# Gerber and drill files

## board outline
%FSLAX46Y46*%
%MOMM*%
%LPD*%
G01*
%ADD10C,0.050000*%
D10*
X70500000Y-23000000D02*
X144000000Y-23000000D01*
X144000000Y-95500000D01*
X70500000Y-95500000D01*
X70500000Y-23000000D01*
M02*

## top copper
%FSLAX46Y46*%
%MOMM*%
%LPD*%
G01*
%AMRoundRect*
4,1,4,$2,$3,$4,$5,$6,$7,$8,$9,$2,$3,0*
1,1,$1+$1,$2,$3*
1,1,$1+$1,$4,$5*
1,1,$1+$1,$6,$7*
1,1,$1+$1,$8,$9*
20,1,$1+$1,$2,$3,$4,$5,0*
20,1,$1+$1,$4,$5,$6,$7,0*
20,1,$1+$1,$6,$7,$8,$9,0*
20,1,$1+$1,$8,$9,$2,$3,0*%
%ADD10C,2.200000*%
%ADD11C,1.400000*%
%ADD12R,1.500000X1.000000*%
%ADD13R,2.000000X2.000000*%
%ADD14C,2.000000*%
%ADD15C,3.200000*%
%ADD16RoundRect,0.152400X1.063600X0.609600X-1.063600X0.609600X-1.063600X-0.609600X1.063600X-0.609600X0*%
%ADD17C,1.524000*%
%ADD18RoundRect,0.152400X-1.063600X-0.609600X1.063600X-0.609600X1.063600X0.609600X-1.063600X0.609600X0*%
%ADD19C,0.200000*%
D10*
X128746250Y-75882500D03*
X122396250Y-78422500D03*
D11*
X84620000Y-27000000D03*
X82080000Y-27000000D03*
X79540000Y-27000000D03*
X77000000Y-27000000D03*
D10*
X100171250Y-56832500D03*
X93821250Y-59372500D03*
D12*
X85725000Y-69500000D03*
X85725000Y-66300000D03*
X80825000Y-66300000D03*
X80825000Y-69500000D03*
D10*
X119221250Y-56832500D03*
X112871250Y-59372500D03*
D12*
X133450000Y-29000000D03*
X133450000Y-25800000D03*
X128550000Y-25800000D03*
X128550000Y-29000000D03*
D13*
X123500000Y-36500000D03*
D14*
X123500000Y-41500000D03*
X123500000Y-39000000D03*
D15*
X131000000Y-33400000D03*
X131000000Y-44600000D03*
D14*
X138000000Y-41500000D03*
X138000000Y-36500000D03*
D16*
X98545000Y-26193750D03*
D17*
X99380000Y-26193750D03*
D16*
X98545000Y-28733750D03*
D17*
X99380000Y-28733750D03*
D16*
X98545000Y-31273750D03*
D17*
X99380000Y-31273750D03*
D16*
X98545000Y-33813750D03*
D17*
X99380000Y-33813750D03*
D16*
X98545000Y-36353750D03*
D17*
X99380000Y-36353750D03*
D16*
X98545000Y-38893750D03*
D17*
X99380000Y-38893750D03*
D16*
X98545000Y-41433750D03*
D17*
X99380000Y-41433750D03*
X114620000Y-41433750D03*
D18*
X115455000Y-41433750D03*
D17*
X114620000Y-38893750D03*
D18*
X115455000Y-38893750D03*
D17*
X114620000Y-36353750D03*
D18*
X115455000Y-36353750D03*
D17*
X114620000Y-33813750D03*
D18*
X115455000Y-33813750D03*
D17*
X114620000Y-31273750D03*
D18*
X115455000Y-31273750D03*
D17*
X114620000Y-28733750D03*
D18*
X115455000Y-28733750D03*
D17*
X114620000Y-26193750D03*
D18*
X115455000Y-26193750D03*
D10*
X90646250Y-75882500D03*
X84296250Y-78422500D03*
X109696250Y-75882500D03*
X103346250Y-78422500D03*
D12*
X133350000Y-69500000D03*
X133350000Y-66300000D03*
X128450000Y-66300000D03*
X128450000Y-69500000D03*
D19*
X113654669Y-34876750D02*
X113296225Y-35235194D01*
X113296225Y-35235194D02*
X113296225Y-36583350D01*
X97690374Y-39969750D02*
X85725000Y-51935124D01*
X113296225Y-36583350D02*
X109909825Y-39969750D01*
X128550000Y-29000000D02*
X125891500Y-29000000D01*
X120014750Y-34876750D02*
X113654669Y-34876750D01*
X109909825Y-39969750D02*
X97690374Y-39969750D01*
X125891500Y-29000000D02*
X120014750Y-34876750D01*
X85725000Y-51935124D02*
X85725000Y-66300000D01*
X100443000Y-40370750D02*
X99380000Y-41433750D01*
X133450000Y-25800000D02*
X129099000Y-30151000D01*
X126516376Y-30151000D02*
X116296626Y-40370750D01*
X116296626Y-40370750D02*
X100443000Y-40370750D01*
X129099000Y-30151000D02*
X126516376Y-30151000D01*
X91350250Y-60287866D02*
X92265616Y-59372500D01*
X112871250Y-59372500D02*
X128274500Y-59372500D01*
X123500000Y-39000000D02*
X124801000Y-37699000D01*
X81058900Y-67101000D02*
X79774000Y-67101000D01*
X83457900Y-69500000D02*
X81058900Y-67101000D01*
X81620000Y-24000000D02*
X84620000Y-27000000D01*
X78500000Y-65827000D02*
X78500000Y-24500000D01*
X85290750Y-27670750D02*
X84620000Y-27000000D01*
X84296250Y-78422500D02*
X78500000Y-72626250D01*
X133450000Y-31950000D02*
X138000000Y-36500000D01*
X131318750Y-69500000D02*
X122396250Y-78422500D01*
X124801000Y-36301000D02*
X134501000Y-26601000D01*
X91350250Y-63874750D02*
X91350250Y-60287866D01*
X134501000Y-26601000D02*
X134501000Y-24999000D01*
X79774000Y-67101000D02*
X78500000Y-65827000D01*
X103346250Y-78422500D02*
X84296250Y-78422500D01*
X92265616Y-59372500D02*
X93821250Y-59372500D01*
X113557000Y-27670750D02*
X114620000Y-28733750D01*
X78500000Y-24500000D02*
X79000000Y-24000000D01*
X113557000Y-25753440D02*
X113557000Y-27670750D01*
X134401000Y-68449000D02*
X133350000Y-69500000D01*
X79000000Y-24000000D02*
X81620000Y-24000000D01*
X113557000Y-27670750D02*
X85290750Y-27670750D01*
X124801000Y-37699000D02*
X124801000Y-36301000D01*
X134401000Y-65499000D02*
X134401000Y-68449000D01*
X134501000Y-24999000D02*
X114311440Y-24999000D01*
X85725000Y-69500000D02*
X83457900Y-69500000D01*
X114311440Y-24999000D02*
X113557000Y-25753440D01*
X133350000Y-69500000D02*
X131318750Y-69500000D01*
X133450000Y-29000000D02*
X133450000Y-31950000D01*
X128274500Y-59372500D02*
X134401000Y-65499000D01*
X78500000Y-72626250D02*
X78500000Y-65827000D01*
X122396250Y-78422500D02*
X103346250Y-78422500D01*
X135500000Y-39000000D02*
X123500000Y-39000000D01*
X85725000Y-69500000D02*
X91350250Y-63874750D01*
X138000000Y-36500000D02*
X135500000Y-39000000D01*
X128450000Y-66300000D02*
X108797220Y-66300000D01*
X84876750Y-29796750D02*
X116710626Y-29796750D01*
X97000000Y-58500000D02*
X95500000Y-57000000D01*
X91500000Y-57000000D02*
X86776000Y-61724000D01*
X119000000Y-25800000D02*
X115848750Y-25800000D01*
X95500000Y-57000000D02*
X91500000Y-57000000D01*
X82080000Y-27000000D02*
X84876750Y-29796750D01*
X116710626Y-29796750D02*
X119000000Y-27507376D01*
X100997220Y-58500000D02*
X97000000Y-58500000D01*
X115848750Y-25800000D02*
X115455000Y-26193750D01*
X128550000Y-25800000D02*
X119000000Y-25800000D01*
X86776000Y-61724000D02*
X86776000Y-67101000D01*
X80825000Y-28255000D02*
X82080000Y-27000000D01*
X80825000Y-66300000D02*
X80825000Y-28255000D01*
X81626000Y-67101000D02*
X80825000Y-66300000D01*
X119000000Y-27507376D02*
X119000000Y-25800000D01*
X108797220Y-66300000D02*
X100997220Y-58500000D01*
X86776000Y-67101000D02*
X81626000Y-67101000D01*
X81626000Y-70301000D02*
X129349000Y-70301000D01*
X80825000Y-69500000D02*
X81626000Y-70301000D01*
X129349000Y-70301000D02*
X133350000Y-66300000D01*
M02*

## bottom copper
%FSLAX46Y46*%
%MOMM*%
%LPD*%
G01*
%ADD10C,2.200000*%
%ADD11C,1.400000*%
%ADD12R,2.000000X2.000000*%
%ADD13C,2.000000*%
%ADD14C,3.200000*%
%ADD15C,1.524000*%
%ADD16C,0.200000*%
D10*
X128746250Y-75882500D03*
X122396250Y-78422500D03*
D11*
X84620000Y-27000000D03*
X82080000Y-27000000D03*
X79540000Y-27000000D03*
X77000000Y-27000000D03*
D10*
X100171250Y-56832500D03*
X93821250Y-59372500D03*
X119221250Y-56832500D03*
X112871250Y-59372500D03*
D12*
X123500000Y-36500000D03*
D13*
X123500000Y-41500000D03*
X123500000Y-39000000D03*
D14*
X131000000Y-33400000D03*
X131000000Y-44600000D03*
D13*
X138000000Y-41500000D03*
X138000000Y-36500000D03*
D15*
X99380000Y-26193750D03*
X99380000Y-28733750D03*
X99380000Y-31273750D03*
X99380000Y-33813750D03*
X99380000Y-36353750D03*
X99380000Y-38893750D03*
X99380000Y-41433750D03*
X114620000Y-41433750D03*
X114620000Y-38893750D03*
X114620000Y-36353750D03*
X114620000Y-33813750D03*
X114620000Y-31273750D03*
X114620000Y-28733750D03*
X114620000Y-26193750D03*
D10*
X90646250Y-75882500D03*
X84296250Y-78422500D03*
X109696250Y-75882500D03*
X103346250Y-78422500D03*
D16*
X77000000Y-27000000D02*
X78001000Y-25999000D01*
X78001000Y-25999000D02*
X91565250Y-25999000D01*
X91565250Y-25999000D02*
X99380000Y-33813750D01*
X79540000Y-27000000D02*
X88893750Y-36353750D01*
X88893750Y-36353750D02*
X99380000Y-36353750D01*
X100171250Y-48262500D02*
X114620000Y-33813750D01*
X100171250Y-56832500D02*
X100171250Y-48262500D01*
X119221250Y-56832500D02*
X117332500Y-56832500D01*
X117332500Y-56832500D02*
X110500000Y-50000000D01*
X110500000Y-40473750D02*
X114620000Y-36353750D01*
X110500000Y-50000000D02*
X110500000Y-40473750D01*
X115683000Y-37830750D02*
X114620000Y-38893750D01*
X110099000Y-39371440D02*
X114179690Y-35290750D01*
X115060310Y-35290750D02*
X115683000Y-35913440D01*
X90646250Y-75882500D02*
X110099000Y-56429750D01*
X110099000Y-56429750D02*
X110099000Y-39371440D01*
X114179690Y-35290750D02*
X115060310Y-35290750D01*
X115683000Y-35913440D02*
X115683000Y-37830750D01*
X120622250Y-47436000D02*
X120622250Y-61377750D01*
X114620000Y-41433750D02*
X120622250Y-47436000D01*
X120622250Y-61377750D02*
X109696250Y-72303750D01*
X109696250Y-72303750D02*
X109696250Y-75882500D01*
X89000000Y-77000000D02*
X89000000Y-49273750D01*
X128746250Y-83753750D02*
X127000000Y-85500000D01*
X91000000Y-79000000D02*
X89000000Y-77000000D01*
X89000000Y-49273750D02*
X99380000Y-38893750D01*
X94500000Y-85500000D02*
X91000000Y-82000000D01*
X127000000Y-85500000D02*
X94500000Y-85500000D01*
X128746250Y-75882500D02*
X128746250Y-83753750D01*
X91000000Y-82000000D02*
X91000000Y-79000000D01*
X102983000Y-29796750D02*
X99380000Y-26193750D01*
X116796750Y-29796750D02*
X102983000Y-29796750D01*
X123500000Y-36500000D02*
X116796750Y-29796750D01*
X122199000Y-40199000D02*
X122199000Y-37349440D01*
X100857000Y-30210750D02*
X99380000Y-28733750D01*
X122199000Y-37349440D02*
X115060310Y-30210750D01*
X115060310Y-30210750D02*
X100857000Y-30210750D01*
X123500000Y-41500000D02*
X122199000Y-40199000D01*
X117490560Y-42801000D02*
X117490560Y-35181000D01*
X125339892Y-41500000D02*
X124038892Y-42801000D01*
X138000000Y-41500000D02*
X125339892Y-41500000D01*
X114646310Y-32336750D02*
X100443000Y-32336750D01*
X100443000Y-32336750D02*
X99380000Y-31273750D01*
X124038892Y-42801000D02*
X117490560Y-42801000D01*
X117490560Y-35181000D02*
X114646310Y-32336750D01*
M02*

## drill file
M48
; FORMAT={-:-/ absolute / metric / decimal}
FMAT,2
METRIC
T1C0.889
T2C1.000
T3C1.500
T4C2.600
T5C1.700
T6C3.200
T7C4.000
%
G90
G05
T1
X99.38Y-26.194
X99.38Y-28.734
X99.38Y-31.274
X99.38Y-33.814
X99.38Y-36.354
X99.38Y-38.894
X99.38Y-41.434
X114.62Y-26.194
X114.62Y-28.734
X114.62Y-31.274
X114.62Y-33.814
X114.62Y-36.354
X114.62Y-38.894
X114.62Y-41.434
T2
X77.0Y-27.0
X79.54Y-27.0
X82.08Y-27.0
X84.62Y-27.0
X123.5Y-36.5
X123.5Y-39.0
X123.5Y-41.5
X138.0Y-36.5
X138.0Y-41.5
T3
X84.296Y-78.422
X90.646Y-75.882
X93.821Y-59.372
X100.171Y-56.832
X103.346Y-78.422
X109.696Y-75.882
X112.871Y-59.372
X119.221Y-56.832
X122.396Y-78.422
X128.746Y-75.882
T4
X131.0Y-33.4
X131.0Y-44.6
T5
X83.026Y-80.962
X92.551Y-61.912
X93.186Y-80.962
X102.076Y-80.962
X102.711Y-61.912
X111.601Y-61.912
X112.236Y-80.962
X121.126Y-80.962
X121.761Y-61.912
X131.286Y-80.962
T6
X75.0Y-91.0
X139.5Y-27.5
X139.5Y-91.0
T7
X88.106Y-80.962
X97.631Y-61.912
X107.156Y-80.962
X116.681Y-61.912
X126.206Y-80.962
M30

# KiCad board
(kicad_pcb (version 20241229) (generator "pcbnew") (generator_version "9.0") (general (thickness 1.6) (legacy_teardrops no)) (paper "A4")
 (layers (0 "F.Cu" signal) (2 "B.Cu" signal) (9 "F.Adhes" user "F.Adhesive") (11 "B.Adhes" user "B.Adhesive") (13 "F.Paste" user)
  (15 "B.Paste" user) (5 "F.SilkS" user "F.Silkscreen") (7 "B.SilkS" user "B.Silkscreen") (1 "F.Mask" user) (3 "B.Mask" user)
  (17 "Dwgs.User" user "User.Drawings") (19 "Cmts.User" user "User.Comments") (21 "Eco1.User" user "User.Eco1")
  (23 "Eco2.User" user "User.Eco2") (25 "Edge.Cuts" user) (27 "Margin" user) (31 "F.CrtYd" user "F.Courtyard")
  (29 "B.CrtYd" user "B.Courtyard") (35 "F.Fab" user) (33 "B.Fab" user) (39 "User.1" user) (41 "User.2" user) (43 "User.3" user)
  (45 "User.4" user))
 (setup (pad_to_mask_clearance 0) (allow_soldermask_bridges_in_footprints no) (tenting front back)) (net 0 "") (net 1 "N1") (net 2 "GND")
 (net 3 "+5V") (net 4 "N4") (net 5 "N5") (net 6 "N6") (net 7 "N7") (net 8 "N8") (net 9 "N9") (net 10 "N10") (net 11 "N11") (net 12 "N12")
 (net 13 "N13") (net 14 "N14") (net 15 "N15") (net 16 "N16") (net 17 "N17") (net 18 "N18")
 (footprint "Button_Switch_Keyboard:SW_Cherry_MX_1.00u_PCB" (layer "F.Cu") (at 128.74625 75.8825)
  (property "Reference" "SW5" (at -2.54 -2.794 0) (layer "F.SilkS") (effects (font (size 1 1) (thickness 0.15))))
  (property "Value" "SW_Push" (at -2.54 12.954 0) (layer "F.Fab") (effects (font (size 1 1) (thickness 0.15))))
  (pad "" np_thru_hole circle (at -7.62 5.08) (size 1.7 1.7) (drill 1.7) (layers "*.Cu" "*.Mask"))
  (pad "" np_thru_hole circle (at -2.54 5.08) (size 4 4) (drill 4) (layers "*.Cu" "*.Mask"))
  (pad "" np_thru_hole circle (at 2.54 5.08) (size 1.7 1.7) (drill 1.7) (layers "*.Cu" "*.Mask"))
  (pad "1" thru_hole circle (at 0 0) (size 2.2 2.2) (drill 1.5) (layers "*.Cu" "*.Mask") (remove_unused_layers no) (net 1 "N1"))
  (pad "2" thru_hole circle (at -6.35 2.54) (size 2.2 2.2) (drill 1.5) (layers "*.Cu" "*.Mask") (remove_unused_layers no) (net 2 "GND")))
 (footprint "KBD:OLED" (layer "F.Cu") (at 80.81 27 180)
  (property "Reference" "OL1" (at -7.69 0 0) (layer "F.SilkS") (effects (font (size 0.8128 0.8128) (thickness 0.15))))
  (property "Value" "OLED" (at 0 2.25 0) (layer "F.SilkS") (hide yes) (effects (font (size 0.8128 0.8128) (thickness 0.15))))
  (pad "1" thru_hole circle (at -3.81 0 180) (size 1.4 1.4) (drill 1) (layers "*.Cu" "*.Mask") (remove_unused_layers no) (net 2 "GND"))
  (pad "2" thru_hole circle (at -1.27 0 180) (size 1.4 1.4) (drill 1) (layers "*.Cu" "*.Mask") (remove_unused_layers no) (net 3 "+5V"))
  (pad "3" thru_hole circle (at 1.27 0 180) (size 1.4 1.4) (drill 1) (layers "*.Cu" "*.Mask") (remove_unused_layers no) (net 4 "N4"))
  (pad "4" thru_hole circle (at 3.81 0 180) (size 1.4 1.4) (drill 1) (layers "*.Cu" "*.Mask") (remove_unused_layers no) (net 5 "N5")))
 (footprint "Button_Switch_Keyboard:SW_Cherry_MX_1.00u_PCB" (layer "F.Cu") (at 100.17125 56.8325)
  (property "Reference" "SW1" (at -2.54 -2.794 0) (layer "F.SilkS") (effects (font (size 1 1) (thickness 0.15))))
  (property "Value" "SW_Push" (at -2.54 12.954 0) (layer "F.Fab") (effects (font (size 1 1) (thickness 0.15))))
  (pad "" np_thru_hole circle (at -7.62 5.08) (size 1.7 1.7) (drill 1.7) (layers "*.Cu" "*.Mask"))
  (pad "" np_thru_hole circle (at -2.54 5.08) (size 4 4) (drill 4) (layers "*.Cu" "*.Mask"))
  (pad "" np_thru_hole circle (at 2.54 5.08) (size 1.7 1.7) (drill 1.7) (layers "*.Cu" "*.Mask"))
  (pad "1" thru_hole circle (at 0 0) (size 2.2 2.2) (drill 1.5) (layers "*.Cu" "*.Mask") (remove_unused_layers no) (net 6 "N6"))
  (pad "2" thru_hole circle (at -6.35 2.54) (size 2.2 2.2) (drill 1.5) (layers "*.Cu" "*.Mask") (remove_unused_layers no) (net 2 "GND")))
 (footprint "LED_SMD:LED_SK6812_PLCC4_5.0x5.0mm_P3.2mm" (layer "F.Cu") (at 83.275 67.9 180)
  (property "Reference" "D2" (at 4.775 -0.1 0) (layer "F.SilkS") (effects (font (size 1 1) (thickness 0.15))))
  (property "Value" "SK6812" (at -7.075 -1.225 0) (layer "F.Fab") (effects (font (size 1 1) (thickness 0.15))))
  (pad "1" smd rect (at -2.45 -1.6) (size 1.5 1) (layers "F.Cu" "F.Mask" "F.Paste") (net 2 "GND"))
  (pad "2" smd rect (at -2.45 1.6) (size 1.5 1) (layers "F.Cu" "F.Mask" "F.Paste") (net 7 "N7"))
  (pad "3" smd rect (at 2.45 1.6) (size 1.5 1) (layers "F.Cu" "F.Mask" "F.Paste") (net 3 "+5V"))
  (pad "4" smd rect (at 2.45 -1.6) (size 1.5 1) (layers "F.Cu" "F.Mask" "F.Paste") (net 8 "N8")))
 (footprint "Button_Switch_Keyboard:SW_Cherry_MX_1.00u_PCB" (layer "F.Cu") (at 119.22125 56.8325)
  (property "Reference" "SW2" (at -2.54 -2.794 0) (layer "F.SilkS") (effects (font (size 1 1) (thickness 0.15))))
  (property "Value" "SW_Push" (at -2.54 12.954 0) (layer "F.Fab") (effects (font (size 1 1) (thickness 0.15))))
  (pad "" np_thru_hole circle (at -7.62 5.08) (size 1.7 1.7) (drill 1.7) (layers "*.Cu" "*.Mask"))
  (pad "" np_thru_hole circle (at -2.54 5.08) (size 4 4) (drill 4) (layers "*.Cu" "*.Mask"))
  (pad "" np_thru_hole circle (at 2.54 5.08) (size 1.7 1.7) (drill 1.7) (layers "*.Cu" "*.Mask"))
  (pad "1" thru_hole circle (at 0 0) (size 2.2 2.2) (drill 1.5) (layers "*.Cu" "*.Mask") (remove_unused_layers no) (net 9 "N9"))
  (pad "2" thru_hole circle (at -6.35 2.54) (size 2.2 2.2) (drill 1.5) (layers "*.Cu" "*.Mask") (remove_unused_layers no) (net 2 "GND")))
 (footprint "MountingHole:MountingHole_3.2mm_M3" (layer "F.Cu") (at 75 91)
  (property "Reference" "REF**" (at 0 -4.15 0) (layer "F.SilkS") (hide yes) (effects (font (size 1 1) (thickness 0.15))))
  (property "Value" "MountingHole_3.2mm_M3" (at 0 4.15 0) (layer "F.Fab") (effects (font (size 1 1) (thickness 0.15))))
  (pad "" np_thru_hole circle (at 0 0) (size 3.2 3.2) (drill 3.2) (layers "*.Cu" "*.Mask")))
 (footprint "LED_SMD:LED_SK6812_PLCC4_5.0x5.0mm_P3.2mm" (layer "F.Cu") (at 131 27.4 180)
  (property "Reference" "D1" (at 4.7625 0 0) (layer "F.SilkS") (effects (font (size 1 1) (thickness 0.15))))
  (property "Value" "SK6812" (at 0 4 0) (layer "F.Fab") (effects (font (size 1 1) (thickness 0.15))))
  (pad "1" smd rect (at -2.45 -1.6) (size 1.5 1) (layers "F.Cu" "F.Mask" "F.Paste") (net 2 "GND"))
  (pad "2" smd rect (at -2.45 1.6) (size 1.5 1) (layers "F.Cu" "F.Mask" "F.Paste") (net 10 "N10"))
  (pad "3" smd rect (at 2.45 1.6) (size 1.5 1) (layers "F.Cu" "F.Mask" "F.Paste") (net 3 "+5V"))
  (pad "4" smd rect (at 2.45 -1.6) (size 1.5 1) (layers "F.Cu" "F.Mask" "F.Paste") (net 7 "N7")))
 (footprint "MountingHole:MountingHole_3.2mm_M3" (layer "F.Cu") (at 139.5 27.5)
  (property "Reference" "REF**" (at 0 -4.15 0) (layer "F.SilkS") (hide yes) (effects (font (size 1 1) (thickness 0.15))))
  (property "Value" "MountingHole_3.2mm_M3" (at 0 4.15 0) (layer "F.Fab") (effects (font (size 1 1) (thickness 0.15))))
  (pad "" np_thru_hole circle (at 0 0) (size 3.2 3.2) (drill 3.2) (layers "*.Cu" "*.Mask")))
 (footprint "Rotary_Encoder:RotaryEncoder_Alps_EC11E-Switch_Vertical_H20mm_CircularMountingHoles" (layer "F.Cu") (at 123.5 36.5)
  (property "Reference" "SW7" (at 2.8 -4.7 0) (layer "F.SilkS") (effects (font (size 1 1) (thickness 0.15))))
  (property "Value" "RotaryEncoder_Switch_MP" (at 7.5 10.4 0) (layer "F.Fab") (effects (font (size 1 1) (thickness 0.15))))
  (pad "A" thru_hole rect (at 0 0) (size 2 2) (drill 1) (layers "*.Cu" "*.Mask") (remove_unused_layers no) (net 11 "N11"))
  (pad "B" thru_hole circle (at 0 5) (size 2 2) (drill 1) (layers "*.Cu" "*.Mask") (remove_unused_layers no) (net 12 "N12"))
  (pad "C" thru_hole circle (at 0 2.5) (size 2 2) (drill 1) (layers "*.Cu" "*.Mask") (remove_unused_layers no) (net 2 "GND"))
  (pad "MP" thru_hole circle (at 7.5 -3.1) (size 3.2 3.2) (drill 2.6) (layers "*.Cu" "*.Mask") (remove_unused_layers no) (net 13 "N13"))
  (pad "MP" thru_hole circle (at 7.5 8.1) (size 3.2 3.2) (drill 2.6) (layers "*.Cu" "*.Mask") (remove_unused_layers no) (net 13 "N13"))
  (pad "S1" thru_hole circle (at 14.5 5) (size 2 2) (drill 1) (layers "*.Cu" "*.Mask") (remove_unused_layers no) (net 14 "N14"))
  (pad "S2" thru_hole circle (at 14.5 0) (size 2 2) (drill 1) (layers "*.Cu" "*.Mask") (remove_unused_layers no) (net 2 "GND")))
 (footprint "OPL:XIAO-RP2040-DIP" (layer "F.Cu") (at 107 33.81375)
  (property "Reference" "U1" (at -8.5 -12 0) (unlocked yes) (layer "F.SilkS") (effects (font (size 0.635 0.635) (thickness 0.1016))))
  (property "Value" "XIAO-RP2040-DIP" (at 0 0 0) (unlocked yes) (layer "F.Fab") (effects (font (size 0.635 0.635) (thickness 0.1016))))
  (pad "1" smd roundrect (at -8.455 -7.62 180) (size 2.432 1.524) (layers "F.Cu" "F.Mask") (roundrect_rratio 0.1) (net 11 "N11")
   (thermal_bridge_angle 45))
  (pad "1" thru_hole circle (at -7.62 -7.62 180) (size 1.524 1.524) (drill 0.889) (layers "*.Cu" "*.Mask") (remove_unused_layers no)
   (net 11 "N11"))
  (pad "2" smd roundrect (at -8.455 -5.08 180) (size 2.432 1.524) (layers "F.Cu" "F.Mask") (roundrect_rratio 0.1) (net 12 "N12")
   (thermal_bridge_angle 45))
  (pad "2" thru_hole circle (at -7.62 -5.08 180) (size 1.524 1.524) (drill 0.889) (layers "*.Cu" "*.Mask") (remove_unused_layers no)
   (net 12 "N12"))
  (pad "3" smd roundrect (at -8.455 -2.54 180) (size 2.432 1.524) (layers "F.Cu" "F.Mask") (roundrect_rratio 0.1) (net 14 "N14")
   (thermal_bridge_angle 45))
  (pad "3" thru_hole circle (at -7.62 -2.54 180) (size 1.524 1.524) (drill 0.889) (layers "*.Cu" "*.Mask") (remove_unused_layers no)
   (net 14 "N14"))
  (pad "4" smd roundrect (at -8.455 0 180) (size 2.432 1.524) (layers "F.Cu" "F.Mask") (roundrect_rratio 0.1) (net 5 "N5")
   (thermal_bridge_angle 45))
  (pad "4" thru_hole circle (at -7.62 0 180) (size 1.524 1.524) (drill 0.889) (layers "*.Cu" "*.Mask") (remove_unused_layers no)
   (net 5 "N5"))
  (pad "5" smd roundrect (at -8.455 2.54 180) (size 2.432 1.524) (layers "F.Cu" "F.Mask") (roundrect_rratio 0.1) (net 4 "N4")
   (thermal_bridge_angle 45))
  (pad "5" thru_hole circle (at -7.62 2.54 180) (size 1.524 1.524) (drill 0.889) (layers "*.Cu" "*.Mask") (remove_unused_layers no)
   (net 4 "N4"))
  (pad "6" smd roundrect (at -8.455 5.08 180) (size 2.432 1.524) (layers "F.Cu" "F.Mask") (roundrect_rratio 0.1) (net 1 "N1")
   (thermal_bridge_angle 45))
  (pad "6" thru_hole circle (at -7.62 5.08 180) (size 1.524 1.524) (drill 0.889) (layers "*.Cu" "*.Mask") (remove_unused_layers no)
   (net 1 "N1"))
  (pad "7" smd roundrect (at -8.455 7.62 180) (size 2.432 1.524) (layers "F.Cu" "F.Mask") (roundrect_rratio 0.1) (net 10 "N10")
   (thermal_bridge_angle 45))
  (pad "7" thru_hole circle (at -7.62 7.62 180) (size 1.524 1.524) (drill 0.889) (layers "*.Cu" "*.Mask") (remove_unused_layers no)
   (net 10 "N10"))
  (pad "8" thru_hole circle (at 7.62 7.62) (size 1.524 1.524) (drill 0.889) (layers "*.Cu" "*.Mask") (remove_unused_layers no)
   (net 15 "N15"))
  (pad "8" smd roundrect (at 8.455 7.62) (size 2.432 1.524) (layers "F.Cu" "F.Mask") (roundrect_rratio 0.1) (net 15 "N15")
   (thermal_bridge_angle 45))
  (pad "9" thru_hole circle (at 7.62 5.08) (size 1.524 1.524) (drill 0.889) (layers "*.Cu" "*.Mask") (remove_unused_layers no)
   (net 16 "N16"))
  (pad "9" smd roundrect (at 8.455 5.08) (size 2.432 1.524) (layers "F.Cu" "F.Mask") (roundrect_rratio 0.1) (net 16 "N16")
   (thermal_bridge_angle 45))
  (pad "10" thru_hole circle (at 7.62 2.54) (size 1.524 1.524) (drill 0.889) (layers "*.Cu" "*.Mask") (remove_unused_layers no) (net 9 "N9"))
  (pad "10" smd roundrect (at 8.455 2.54) (size 2.432 1.524) (layers "F.Cu" "F.Mask") (roundrect_rratio 0.1) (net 9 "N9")
   (thermal_bridge_angle 45))
  (pad "11" thru_hole circle (at 7.62 0) (size 1.524 1.524) (drill 0.889) (layers "*.Cu" "*.Mask") (remove_unused_layers no) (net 6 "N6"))
  (pad "11" smd roundrect (at 8.455 0) (size 2.432 1.524) (layers "F.Cu" "F.Mask") (roundrect_rratio 0.1) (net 6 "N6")
   (thermal_bridge_angle 45))
  (pad "12" thru_hole circle (at 7.62 -2.54) (size 1.524 1.524) (drill 0.889) (layers "*.Cu" "*.Mask") (remove_unused_layers no)
   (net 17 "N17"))
  (pad "12" smd roundrect (at 8.455 -2.54) (size 2.432 1.524) (layers "F.Cu" "F.Mask") (roundrect_rratio 0.1) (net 17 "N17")
   (thermal_bridge_angle 45))
  (pad "13" thru_hole circle (at 7.62 -5.08) (size 1.524 1.524) (drill 0.889) (layers "*.Cu" "*.Mask") (remove_unused_layers no)
   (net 2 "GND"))
  (pad "13" smd roundrect (at 8.455 -5.08) (size 2.432 1.524) (layers "F.Cu" "F.Mask") (roundrect_rratio 0.1) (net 2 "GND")
   (thermal_bridge_angle 45))
  (pad "14" thru_hole circle (at 7.62 -7.62) (size 1.524 1.524) (drill 0.889) (layers "*.Cu" "*.Mask") (remove_unused_layers no)
   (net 3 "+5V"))
  (pad "14" smd roundrect (at 8.455 -7.62) (size 2.432 1.524) (layers "F.Cu" "F.Mask") (roundrect_rratio 0.1) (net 3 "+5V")
   (thermal_bridge_angle 45)))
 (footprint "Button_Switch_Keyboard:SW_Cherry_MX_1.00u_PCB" (layer "F.Cu") (at 90.64625 75.8825)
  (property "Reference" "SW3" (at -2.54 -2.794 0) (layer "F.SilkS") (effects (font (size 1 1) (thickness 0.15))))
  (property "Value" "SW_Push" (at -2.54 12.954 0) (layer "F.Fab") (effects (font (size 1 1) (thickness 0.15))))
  (pad "" np_thru_hole circle (at -7.62 5.08) (size 1.7 1.7) (drill 1.7) (layers "*.Cu" "*.Mask"))
  (pad "" np_thru_hole circle (at -2.54 5.08) (size 4 4) (drill 4) (layers "*.Cu" "*.Mask"))
  (pad "" np_thru_hole circle (at 2.54 5.08) (size 1.7 1.7) (drill 1.7) (layers "*.Cu" "*.Mask"))
  (pad "1" thru_hole circle (at 0 0) (size 2.2 2.2) (drill 1.5) (layers "*.Cu" "*.Mask") (remove_unused_layers no) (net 16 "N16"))
  (pad "2" thru_hole circle (at -6.35 2.54) (size 2.2 2.2) (drill 1.5) (layers "*.Cu" "*.Mask") (remove_unused_layers no) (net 2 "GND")))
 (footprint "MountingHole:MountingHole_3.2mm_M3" (layer "F.Cu") (at 139.5 91)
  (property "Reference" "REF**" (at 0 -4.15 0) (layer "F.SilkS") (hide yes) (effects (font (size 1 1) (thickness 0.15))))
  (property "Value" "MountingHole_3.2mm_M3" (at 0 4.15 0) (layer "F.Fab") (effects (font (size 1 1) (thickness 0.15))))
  (pad "" np_thru_hole circle (at 0 0) (size 3.2 3.2) (drill 3.2) (layers "*.Cu" "*.Mask")))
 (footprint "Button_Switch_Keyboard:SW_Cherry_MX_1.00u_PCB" (layer "F.Cu") (at 109.69625 75.8825)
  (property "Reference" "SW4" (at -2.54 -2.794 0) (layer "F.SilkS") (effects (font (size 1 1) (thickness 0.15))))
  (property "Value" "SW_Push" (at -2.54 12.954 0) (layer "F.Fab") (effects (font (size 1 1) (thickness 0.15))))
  (pad "" np_thru_hole circle (at -7.62 5.08) (size 1.7 1.7) (drill 1.7) (layers "*.Cu" "*.Mask"))
  (pad "" np_thru_hole circle (at -2.54 5.08) (size 4 4) (drill 4) (layers "*.Cu" "*.Mask"))
  (pad "" np_thru_hole circle (at 2.54 5.08) (size 1.7 1.7) (drill 1.7) (layers "*.Cu" "*.Mask"))
  (pad "1" thru_hole circle (at 0 0) (size 2.2 2.2) (drill 1.5) (layers "*.Cu" "*.Mask") (remove_unused_layers no) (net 15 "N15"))
  (pad "2" thru_hole circle (at -6.35 2.54) (size 2.2 2.2) (drill 1.5) (layers "*.Cu" "*.Mask") (remove_unused_layers no) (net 2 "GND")))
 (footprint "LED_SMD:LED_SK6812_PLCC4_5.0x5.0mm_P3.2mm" (layer "F.Cu") (at 130.9 67.9 180)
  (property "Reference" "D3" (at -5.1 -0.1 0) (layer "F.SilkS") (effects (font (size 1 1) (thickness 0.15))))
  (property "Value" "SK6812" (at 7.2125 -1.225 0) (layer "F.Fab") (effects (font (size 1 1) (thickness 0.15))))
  (pad "1" smd rect (at -2.45 -1.6) (size 1.5 1) (layers "F.Cu" "F.Mask" "F.Paste") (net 2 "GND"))
  (pad "2" smd rect (at -2.45 1.6) (size 1.5 1) (layers "F.Cu" "F.Mask" "F.Paste") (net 8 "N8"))
  (pad "3" smd rect (at 2.45 1.6) (size 1.5 1) (layers "F.Cu" "F.Mask" "F.Paste") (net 3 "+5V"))
  (pad "4" smd rect (at 2.45 -1.6) (size 1.5 1) (layers "F.Cu" "F.Mask" "F.Paste") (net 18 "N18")))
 (gr_rect (start 70.5 23) (end 144 95.5) (stroke (width 0.05) (type default)) (fill no) (layer "Edge.Cuts"))
 (segment (start 113.654669 34.87675) (end 113.296225 35.235194) (width 0.2) (layer "F.Cu") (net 7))
 (segment (start 113.296225 35.235194) (end 113.296225 36.58335) (width 0.2) (layer "F.Cu") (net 7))
 (segment (start 97.690374 39.96975) (end 85.725 51.935124) (width 0.2) (layer "F.Cu") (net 7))
 (segment (start 113.296225 36.58335) (end 109.909825 39.96975) (width 0.2) (layer "F.Cu") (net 7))
 (segment (start 128.55 29) (end 125.8915 29) (width 0.2) (layer "F.Cu") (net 7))
 (segment (start 120.01475 34.87675) (end 113.654669 34.87675) (width 0.2) (layer "F.Cu") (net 7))
 (segment (start 109.909825 39.96975) (end 97.690374 39.96975) (width 0.2) (layer "F.Cu") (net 7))
 (segment (start 125.8915 29) (end 120.01475 34.87675) (width 0.2) (layer "F.Cu") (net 7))
 (segment (start 85.725 51.935124) (end 85.725 66.3) (width 0.2) (layer "F.Cu") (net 7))
 (segment (start 100.443 40.37075) (end 99.38 41.43375) (width 0.2) (layer "F.Cu") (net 10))
 (segment (start 133.45 25.8) (end 129.099 30.151) (width 0.2) (layer "F.Cu") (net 10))
 (segment (start 126.516376 30.151) (end 116.296626 40.37075) (width 0.2) (layer "F.Cu") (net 10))
 (segment (start 116.296626 40.37075) (end 100.443 40.37075) (width 0.2) (layer "F.Cu") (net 10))
 (segment (start 129.099 30.151) (end 126.516376 30.151) (width 0.2) (layer "F.Cu") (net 10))
 (segment (start 91.35025 60.287866) (end 92.265616 59.3725) (width 0.2) (layer "F.Cu") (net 2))
 (segment (start 112.87125 59.3725) (end 128.2745 59.3725) (width 0.2) (layer "F.Cu") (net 2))
 (segment (start 123.5 39) (end 124.801 37.699) (width 0.2) (layer "F.Cu") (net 2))
 (segment (start 81.0589 67.101) (end 79.774 67.101) (width 0.2) (layer "F.Cu") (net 2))
 (segment (start 83.4579 69.5) (end 81.0589 67.101) (width 0.2) (layer "F.Cu") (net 2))
 (segment (start 81.62 24) (end 84.62 27) (width 0.2) (layer "F.Cu") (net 2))
 (segment (start 78.5 65.827) (end 78.5 24.5) (width 0.2) (layer "F.Cu") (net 2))
 (segment (start 85.29075 27.67075) (end 84.62 27) (width 0.2) (layer "F.Cu") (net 2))
 (segment (start 84.29625 78.4225) (end 78.5 72.62625) (width 0.2) (layer "F.Cu") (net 2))
 (segment (start 133.45 31.95) (end 138 36.5) (width 0.2) (layer "F.Cu") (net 2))
 (segment (start 131.31875 69.5) (end 122.39625 78.4225) (width 0.2) (layer "F.Cu") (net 2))
 (segment (start 124.801 36.301) (end 134.501 26.601) (width 0.2) (layer "F.Cu") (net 2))
 (segment (start 91.35025 63.87475) (end 91.35025 60.287866) (width 0.2) (layer "F.Cu") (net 2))
 (segment (start 134.501 26.601) (end 134.501 24.999) (width 0.2) (layer "F.Cu") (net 2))
 (segment (start 79.774 67.101) (end 78.5 65.827) (width 0.2) (layer "F.Cu") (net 2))
 (segment (start 103.34625 78.4225) (end 84.29625 78.4225) (width 0.2) (layer "F.Cu") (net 2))
 (segment (start 92.265616 59.3725) (end 93.82125 59.3725) (width 0.2) (layer "F.Cu") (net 2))
 (segment (start 113.557 27.67075) (end 114.62 28.73375) (width 0.2) (layer "F.Cu") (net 2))
 (segment (start 78.5 24.5) (end 79 24) (width 0.2) (layer "F.Cu") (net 2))
 (segment (start 113.557 25.75344) (end 113.557 27.67075) (width 0.2) (layer "F.Cu") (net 2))
 (segment (start 134.401 68.449) (end 133.35 69.5) (width 0.2) (layer "F.Cu") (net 2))
 (segment (start 79 24) (end 81.62 24) (width 0.2) (layer "F.Cu") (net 2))
 (segment (start 113.557 27.67075) (end 85.29075 27.67075) (width 0.2) (layer "F.Cu") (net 2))
 (segment (start 124.801 37.699) (end 124.801 36.301) (width 0.2) (layer "F.Cu") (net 2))
 (segment (start 134.401 65.499) (end 134.401 68.449) (width 0.2) (layer "F.Cu") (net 2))
 (segment (start 134.501 24.999) (end 114.31144 24.999) (width 0.2) (layer "F.Cu") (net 2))
 (segment (start 85.725 69.5) (end 83.4579 69.5) (width 0.2) (layer "F.Cu") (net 2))
 (segment (start 114.31144 24.999) (end 113.557 25.75344) (width 0.2) (layer "F.Cu") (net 2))
 (segment (start 133.35 69.5) (end 131.31875 69.5) (width 0.2) (layer "F.Cu") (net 2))
 (segment (start 133.45 29) (end 133.45 31.95) (width 0.2) (layer "F.Cu") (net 2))
 (segment (start 128.2745 59.3725) (end 134.401 65.499) (width 0.2) (layer "F.Cu") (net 2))
 (segment (start 78.5 72.62625) (end 78.5 65.827) (width 0.2) (layer "F.Cu") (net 2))
 (segment (start 122.39625 78.4225) (end 103.34625 78.4225) (width 0.2) (layer "F.Cu") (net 2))
 (segment (start 135.5 39) (end 123.5 39) (width 0.2) (layer "F.Cu") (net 2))
 (segment (start 85.725 69.5) (end 91.35025 63.87475) (width 0.2) (layer "F.Cu") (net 2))
 (segment (start 138 36.5) (end 135.5 39) (width 0.2) (layer "F.Cu") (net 2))
 (segment (start 128.45 66.3) (end 108.79722 66.3) (width 0.2) (layer "F.Cu") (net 3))
 (segment (start 84.87675 29.79675) (end 116.710626 29.79675) (width 0.2) (layer "F.Cu") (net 3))
 (segment (start 97 58.5) (end 95.5 57) (width 0.2) (layer "F.Cu") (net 3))
 (segment (start 91.5 57) (end 86.776 61.724) (width 0.2) (layer "F.Cu") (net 3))
 (segment (start 119 25.8) (end 115.84875 25.8) (width 0.2) (layer "F.Cu") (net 3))
 (segment (start 95.5 57) (end 91.5 57) (width 0.2) (layer "F.Cu") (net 3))
 (segment (start 82.08 27) (end 84.87675 29.79675) (width 0.2) (layer "F.Cu") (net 3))
 (segment (start 116.710626 29.79675) (end 119 27.507376) (width 0.2) (layer "F.Cu") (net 3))
 (segment (start 100.99722 58.5) (end 97 58.5) (width 0.2) (layer "F.Cu") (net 3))
 (segment (start 115.84875 25.8) (end 115.455 26.19375) (width 0.2) (layer "F.Cu") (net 3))
 (segment (start 128.55 25.8) (end 119 25.8) (width 0.2) (layer "F.Cu") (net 3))
 (segment (start 86.776 61.724) (end 86.776 67.101) (width 0.2) (layer "F.Cu") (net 3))
 (segment (start 80.825 28.255) (end 82.08 27) (width 0.2) (layer "F.Cu") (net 3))
 (segment (start 80.825 66.3) (end 80.825 28.255) (width 0.2) (layer "F.Cu") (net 3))
 (segment (start 81.626 67.101) (end 80.825 66.3) (width 0.2) (layer "F.Cu") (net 3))
 (segment (start 119 27.507376) (end 119 25.8) (width 0.2) (layer "F.Cu") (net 3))
 (segment (start 108.79722 66.3) (end 100.99722 58.5) (width 0.2) (layer "F.Cu") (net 3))
 (segment (start 86.776 67.101) (end 81.626 67.101) (width 0.2) (layer "F.Cu") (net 3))
 (segment (start 81.626 70.301) (end 129.349 70.301) (width 0.2) (layer "F.Cu") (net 8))
 (segment (start 80.825 69.5) (end 81.626 70.301) (width 0.2) (layer "F.Cu") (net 8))
 (segment (start 129.349 70.301) (end 133.35 66.3) (width 0.2) (layer "F.Cu") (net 8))
 (segment (start 77 27) (end 78.001 25.999) (width 0.2) (layer "B.Cu") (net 5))
 (segment (start 78.001 25.999) (end 91.56525 25.999) (width 0.2) (layer "B.Cu") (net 5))
 (segment (start 91.56525 25.999) (end 99.38 33.81375) (width 0.2) (layer "B.Cu") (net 5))
 (segment (start 79.54 27) (end 88.89375 36.35375) (width 0.2) (layer "B.Cu") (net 4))
 (segment (start 88.89375 36.35375) (end 99.38 36.35375) (width 0.2) (layer "B.Cu") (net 4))
 (segment (start 100.17125 48.2625) (end 114.62 33.81375) (width 0.2) (layer "B.Cu") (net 6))
 (segment (start 100.17125 56.8325) (end 100.17125 48.2625) (width 0.2) (layer "B.Cu") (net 6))
 (segment (start 119.22125 56.8325) (end 117.3325 56.8325) (width 0.2) (layer "B.Cu") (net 9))
 (segment (start 117.3325 56.8325) (end 110.5 50) (width 0.2) (layer "B.Cu") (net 9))
 (segment (start 110.5 40.47375) (end 114.62 36.35375) (width 0.2) (layer "B.Cu") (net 9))
 (segment (start 110.5 50) (end 110.5 40.47375) (width 0.2) (layer "B.Cu") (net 9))
 (segment (start 115.683 37.83075) (end 114.62 38.89375) (width 0.2) (layer "B.Cu") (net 16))
 (segment (start 110.099 39.37144) (end 114.17969 35.29075) (width 0.2) (layer "B.Cu") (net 16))
 (segment (start 115.06031 35.29075) (end 115.683 35.91344) (width 0.2) (layer "B.Cu") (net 16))
 (segment (start 90.64625 75.8825) (end 110.099 56.42975) (width 0.2) (layer "B.Cu") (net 16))
 (segment (start 110.099 56.42975) (end 110.099 39.37144) (width 0.2) (layer "B.Cu") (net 16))
 (segment (start 114.17969 35.29075) (end 115.06031 35.29075) (width 0.2) (layer "B.Cu") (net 16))
 (segment (start 115.683 35.91344) (end 115.683 37.83075) (width 0.2) (layer "B.Cu") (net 16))
 (segment (start 120.62225 47.436) (end 120.62225 61.37775) (width 0.2) (layer "B.Cu") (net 15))
 (segment (start 114.62 41.43375) (end 120.62225 47.436) (width 0.2) (layer "B.Cu") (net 15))
 (segment (start 120.62225 61.37775) (end 109.69625 72.30375) (width 0.2) (layer "B.Cu") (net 15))
 (segment (start 109.69625 72.30375) (end 109.69625 75.8825) (width 0.2) (layer "B.Cu") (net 15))
 (segment (start 89 77) (end 89 49.27375) (width 0.2) (layer "B.Cu") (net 1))
 (segment (start 128.74625 83.75375) (end 127 85.5) (width 0.2) (layer "B.Cu") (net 1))
 (segment (start 91 79) (end 89 77) (width 0.2) (layer "B.Cu") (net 1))
 (segment (start 89 49.27375) (end 99.38 38.89375) (width 0.2) (layer "B.Cu") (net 1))
 (segment (start 94.5 85.5) (end 91 82) (width 0.2) (layer "B.Cu") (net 1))
 (segment (start 127 85.5) (end 94.5 85.5) (width 0.2) (layer "B.Cu") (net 1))
 (segment (start 128.74625 75.8825) (end 128.74625 83.75375) (width 0.2) (layer "B.Cu") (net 1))
 (segment (start 91 82) (end 91 79) (width 0.2) (layer "B.Cu") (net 1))
 (segment (start 102.983 29.79675) (end 99.38 26.19375) (width 0.2) (layer "B.Cu") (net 11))
 (segment (start 116.79675 29.79675) (end 102.983 29.79675) (width 0.2) (layer "B.Cu") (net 11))
 (segment (start 123.5 36.5) (end 116.79675 29.79675) (width 0.2) (layer "B.Cu") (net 11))
 (segment (start 122.199 40.199) (end 122.199 37.34944) (width 0.2) (layer "B.Cu") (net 12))
 (segment (start 100.857 30.21075) (end 99.38 28.73375) (width 0.2) (layer "B.Cu") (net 12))
 (segment (start 122.199 37.34944) (end 115.06031 30.21075) (width 0.2) (layer "B.Cu") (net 12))
 (segment (start 115.06031 30.21075) (end 100.857 30.21075) (width 0.2) (layer "B.Cu") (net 12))
 (segment (start 123.5 41.5) (end 122.199 40.199) (width 0.2) (layer "B.Cu") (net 12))
 (segment (start 117.49056 42.801) (end 117.49056 35.181) (width 0.2) (layer "B.Cu") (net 14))
 (segment (start 125.339892 41.5) (end 124.038892 42.801) (width 0.2) (layer "B.Cu") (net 14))
 (segment (start 138 41.5) (end 125.339892 41.5) (width 0.2) (layer "B.Cu") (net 14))
 (segment (start 114.64631 32.33675) (end 100.443 32.33675) (width 0.2) (layer "B.Cu") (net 14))
 (segment (start 100.443 32.33675) (end 99.38 31.27375) (width 0.2) (layer "B.Cu") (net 14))
 (segment (start 124.038892 42.801) (end 117.49056 42.801) (width 0.2) (layer "B.Cu") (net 14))
 (segment (start 117.49056 35.181) (end 114.64631 32.33675) (width 0.2) (layer "B.Cu") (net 14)))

